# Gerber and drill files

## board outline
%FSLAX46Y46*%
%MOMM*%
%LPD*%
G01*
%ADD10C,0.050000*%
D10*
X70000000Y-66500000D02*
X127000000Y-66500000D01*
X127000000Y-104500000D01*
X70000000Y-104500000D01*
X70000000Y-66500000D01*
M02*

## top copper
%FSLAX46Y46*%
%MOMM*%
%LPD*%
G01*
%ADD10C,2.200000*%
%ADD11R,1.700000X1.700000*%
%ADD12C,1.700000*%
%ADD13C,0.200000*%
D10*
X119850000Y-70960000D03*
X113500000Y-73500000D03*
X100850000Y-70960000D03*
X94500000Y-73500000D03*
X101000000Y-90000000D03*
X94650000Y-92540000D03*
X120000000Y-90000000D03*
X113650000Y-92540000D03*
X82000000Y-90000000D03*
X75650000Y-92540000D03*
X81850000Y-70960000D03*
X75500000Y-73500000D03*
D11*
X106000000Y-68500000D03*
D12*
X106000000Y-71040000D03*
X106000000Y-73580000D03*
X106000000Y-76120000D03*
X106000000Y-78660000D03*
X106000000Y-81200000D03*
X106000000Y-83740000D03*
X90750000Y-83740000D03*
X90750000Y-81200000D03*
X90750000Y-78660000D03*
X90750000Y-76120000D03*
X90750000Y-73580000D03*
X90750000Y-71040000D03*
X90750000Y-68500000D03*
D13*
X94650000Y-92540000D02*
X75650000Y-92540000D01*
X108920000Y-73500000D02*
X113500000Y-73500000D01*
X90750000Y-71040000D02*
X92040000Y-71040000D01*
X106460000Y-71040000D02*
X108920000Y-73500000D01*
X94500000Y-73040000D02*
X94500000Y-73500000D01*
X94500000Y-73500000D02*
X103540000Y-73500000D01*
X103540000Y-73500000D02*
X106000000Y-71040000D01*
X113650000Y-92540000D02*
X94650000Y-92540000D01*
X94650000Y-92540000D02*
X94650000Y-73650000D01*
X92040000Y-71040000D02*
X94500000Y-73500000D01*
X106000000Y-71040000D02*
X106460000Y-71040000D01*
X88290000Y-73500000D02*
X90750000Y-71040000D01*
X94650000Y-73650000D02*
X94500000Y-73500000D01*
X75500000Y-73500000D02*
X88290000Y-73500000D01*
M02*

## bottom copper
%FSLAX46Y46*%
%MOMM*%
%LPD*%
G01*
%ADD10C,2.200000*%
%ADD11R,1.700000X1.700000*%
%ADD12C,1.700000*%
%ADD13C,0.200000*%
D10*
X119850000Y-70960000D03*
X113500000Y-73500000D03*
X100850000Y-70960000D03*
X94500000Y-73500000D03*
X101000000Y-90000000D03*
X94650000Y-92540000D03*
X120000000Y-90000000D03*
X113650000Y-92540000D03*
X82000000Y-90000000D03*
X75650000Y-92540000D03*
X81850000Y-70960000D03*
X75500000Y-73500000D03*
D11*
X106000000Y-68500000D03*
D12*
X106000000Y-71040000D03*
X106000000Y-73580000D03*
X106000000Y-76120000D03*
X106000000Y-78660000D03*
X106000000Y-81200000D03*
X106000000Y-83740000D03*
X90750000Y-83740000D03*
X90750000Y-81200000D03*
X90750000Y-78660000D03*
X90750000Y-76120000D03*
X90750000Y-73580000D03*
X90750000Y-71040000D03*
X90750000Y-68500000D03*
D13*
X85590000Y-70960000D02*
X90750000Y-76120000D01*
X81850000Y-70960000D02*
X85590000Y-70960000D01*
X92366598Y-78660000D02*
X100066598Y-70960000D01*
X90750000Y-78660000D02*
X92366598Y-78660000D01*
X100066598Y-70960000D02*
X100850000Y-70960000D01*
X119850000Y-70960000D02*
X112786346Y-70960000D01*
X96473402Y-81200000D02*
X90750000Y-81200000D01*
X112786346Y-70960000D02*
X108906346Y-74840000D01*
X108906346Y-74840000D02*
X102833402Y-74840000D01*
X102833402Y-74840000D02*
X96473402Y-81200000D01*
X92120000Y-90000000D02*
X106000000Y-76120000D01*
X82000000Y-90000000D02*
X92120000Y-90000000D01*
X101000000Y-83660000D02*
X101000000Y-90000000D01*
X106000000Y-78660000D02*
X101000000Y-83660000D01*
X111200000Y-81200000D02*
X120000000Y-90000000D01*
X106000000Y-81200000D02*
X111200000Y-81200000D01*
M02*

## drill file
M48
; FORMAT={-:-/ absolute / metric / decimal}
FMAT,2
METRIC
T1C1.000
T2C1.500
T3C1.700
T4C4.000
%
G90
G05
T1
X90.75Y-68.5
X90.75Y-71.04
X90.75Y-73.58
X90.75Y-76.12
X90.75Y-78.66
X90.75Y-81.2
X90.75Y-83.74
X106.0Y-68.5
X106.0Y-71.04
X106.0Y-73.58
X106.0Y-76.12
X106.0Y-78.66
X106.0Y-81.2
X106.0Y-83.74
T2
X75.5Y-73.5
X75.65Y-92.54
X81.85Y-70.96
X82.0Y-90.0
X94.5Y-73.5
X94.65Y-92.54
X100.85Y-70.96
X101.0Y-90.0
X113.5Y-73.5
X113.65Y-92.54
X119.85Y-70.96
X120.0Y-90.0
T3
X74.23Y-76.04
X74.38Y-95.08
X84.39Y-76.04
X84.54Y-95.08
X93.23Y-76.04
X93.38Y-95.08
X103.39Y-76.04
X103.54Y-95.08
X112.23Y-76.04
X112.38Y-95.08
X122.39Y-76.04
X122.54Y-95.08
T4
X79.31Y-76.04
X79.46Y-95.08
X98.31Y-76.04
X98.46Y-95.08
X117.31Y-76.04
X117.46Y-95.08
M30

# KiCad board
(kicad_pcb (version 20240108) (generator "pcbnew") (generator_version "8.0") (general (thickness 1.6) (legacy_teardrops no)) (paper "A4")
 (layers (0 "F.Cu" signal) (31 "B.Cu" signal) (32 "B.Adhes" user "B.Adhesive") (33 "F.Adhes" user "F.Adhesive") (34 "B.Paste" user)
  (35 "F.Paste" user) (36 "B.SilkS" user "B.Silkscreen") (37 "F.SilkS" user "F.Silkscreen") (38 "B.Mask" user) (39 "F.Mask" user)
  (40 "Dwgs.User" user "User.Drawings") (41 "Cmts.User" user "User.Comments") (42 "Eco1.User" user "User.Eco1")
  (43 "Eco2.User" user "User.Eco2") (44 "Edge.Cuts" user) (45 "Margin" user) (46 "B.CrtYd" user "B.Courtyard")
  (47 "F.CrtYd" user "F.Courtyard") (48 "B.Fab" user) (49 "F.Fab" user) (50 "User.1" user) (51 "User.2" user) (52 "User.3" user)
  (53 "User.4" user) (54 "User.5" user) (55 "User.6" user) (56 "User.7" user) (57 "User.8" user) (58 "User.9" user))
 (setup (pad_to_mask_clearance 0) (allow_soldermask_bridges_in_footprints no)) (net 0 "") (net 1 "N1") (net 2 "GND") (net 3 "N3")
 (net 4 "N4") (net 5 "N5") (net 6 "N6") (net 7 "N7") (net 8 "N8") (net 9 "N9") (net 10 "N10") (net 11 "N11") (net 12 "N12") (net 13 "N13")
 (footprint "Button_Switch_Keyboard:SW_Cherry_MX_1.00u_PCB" (layer "F.Cu") (at 119.85 70.96)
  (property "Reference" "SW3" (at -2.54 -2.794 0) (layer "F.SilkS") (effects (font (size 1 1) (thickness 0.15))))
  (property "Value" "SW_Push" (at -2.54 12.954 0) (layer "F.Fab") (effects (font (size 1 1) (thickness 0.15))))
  (pad "" np_thru_hole circle (at -7.62 5.08) (size 1.7 1.7) (drill 1.7) (layers "*.Cu" "*.Mask"))
  (pad "" np_thru_hole circle (at -2.54 5.08) (size 4 4) (drill 4) (layers "*.Cu" "*.Mask"))
  (pad "" np_thru_hole circle (at 2.54 5.08) (size 1.7 1.7) (drill 1.7) (layers "*.Cu" "*.Mask"))
  (pad "1" thru_hole circle (at 0 0) (size 2.2 2.2) (drill 1.5) (layers "*.Cu" "*.Mask") (remove_unused_layers no) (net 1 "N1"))
  (pad "2" thru_hole circle (at -6.35 2.54) (size 2.2 2.2) (drill 1.5) (layers "*.Cu" "*.Mask") (remove_unused_layers no) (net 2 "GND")))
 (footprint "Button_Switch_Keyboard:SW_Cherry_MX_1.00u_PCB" (layer "F.Cu") (at 100.85 70.96)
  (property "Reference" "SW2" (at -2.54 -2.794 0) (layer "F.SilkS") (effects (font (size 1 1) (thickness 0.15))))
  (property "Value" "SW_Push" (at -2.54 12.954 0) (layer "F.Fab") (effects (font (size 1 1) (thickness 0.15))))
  (pad "" np_thru_hole circle (at -7.62 5.08) (size 1.7 1.7) (drill 1.7) (layers "*.Cu" "*.Mask"))
  (pad "" np_thru_hole circle (at -2.54 5.08) (size 4 4) (drill 4) (layers "*.Cu" "*.Mask"))
  (pad "" np_thru_hole circle (at 2.54 5.08) (size 1.7 1.7) (drill 1.7) (layers "*.Cu" "*.Mask"))
  (pad "1" thru_hole circle (at 0 0) (size 2.2 2.2) (drill 1.5) (layers "*.Cu" "*.Mask") (remove_unused_layers no) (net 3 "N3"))
  (pad "2" thru_hole circle (at -6.35 2.54) (size 2.2 2.2) (drill 1.5) (layers "*.Cu" "*.Mask") (remove_unused_layers no) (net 2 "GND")))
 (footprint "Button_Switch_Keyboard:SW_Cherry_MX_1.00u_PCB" (layer "F.Cu") (at 101 90)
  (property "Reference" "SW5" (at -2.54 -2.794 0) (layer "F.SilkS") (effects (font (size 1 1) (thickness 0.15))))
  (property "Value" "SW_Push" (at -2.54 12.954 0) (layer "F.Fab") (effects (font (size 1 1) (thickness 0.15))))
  (pad "" np_thru_hole circle (at -7.62 5.08) (size 1.7 1.7) (drill 1.7) (layers "*.Cu" "*.Mask"))
  (pad "" np_thru_hole circle (at -2.54 5.08) (size 4 4) (drill 4) (layers "*.Cu" "*.Mask"))
  (pad "" np_thru_hole circle (at 2.54 5.08) (size 1.7 1.7) (drill 1.7) (layers "*.Cu" "*.Mask"))
  (pad "1" thru_hole circle (at 0 0) (size 2.2 2.2) (drill 1.5) (layers "*.Cu" "*.Mask") (remove_unused_layers no) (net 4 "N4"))
  (pad "2" thru_hole circle (at -6.35 2.54) (size 2.2 2.2) (drill 1.5) (layers "*.Cu" "*.Mask") (remove_unused_layers no) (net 2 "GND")))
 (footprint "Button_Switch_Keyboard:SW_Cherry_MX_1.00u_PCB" (layer "F.Cu") (at 120 90)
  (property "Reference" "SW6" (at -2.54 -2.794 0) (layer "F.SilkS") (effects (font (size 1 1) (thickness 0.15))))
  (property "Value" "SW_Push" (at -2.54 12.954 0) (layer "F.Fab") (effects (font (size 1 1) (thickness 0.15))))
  (pad "" np_thru_hole circle (at -7.62 5.08) (size 1.7 1.7) (drill 1.7) (layers "*.Cu" "*.Mask"))
  (pad "" np_thru_hole circle (at -2.54 5.08) (size 4 4) (drill 4) (layers "*.Cu" "*.Mask"))
  (pad "" np_thru_hole circle (at 2.54 5.08) (size 1.7 1.7) (drill 1.7) (layers "*.Cu" "*.Mask"))
  (pad "1" thru_hole circle (at 0 0) (size 2.2 2.2) (drill 1.5) (layers "*.Cu" "*.Mask") (remove_unused_layers no) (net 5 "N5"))
  (pad "2" thru_hole circle (at -6.35 2.54) (size 2.2 2.2) (drill 1.5) (layers "*.Cu" "*.Mask") (remove_unused_layers no) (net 2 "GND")))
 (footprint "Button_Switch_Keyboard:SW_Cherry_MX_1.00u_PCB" (layer "F.Cu") (at 82 90)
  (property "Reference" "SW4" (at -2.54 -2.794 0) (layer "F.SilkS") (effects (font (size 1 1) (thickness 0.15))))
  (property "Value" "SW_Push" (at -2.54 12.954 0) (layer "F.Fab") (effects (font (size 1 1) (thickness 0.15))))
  (pad "" np_thru_hole circle (at -7.62 5.08) (size 1.7 1.7) (drill 1.7) (layers "*.Cu" "*.Mask"))
  (pad "" np_thru_hole circle (at -2.54 5.08) (size 4 4) (drill 4) (layers "*.Cu" "*.Mask"))
  (pad "" np_thru_hole circle (at 2.54 5.08) (size 1.7 1.7) (drill 1.7) (layers "*.Cu" "*.Mask"))
  (pad "1" thru_hole circle (at 0 0) (size 2.2 2.2) (drill 1.5) (layers "*.Cu" "*.Mask") (remove_unused_layers no) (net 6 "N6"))
  (pad "2" thru_hole circle (at -6.35 2.54) (size 2.2 2.2) (drill 1.5) (layers "*.Cu" "*.Mask") (remove_unused_layers no) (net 2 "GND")))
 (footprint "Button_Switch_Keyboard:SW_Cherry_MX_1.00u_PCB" (layer "F.Cu") (at 81.85 70.96)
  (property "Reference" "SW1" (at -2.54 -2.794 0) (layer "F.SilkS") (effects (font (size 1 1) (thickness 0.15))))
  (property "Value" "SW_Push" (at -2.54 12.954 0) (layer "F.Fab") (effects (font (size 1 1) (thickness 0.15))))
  (pad "" np_thru_hole circle (at -7.62 5.08) (size 1.7 1.7) (drill 1.7) (layers "*.Cu" "*.Mask"))
  (pad "" np_thru_hole circle (at -2.54 5.08) (size 4 4) (drill 4) (layers "*.Cu" "*.Mask"))
  (pad "" np_thru_hole circle (at 2.54 5.08) (size 1.7 1.7) (drill 1.7) (layers "*.Cu" "*.Mask"))
  (pad "1" thru_hole circle (at 0 0) (size 2.2 2.2) (drill 1.5) (layers "*.Cu" "*.Mask") (remove_unused_layers no) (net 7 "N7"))
  (pad "2" thru_hole circle (at -6.35 2.54) (size 2.2 2.2) (drill 1.5) (layers "*.Cu" "*.Mask") (remove_unused_layers no) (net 2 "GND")))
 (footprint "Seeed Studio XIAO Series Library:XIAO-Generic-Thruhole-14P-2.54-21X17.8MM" (layer "B.Cu") (at 98.375 76.12 180)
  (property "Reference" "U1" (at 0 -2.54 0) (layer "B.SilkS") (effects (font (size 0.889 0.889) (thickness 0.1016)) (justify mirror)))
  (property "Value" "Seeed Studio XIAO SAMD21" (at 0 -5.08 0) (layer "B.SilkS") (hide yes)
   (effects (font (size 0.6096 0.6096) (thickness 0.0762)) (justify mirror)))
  (pad "1" thru_hole rect (at -7.625 7.62 180) (size 1.7 1.7) (drill 1) (layers "*.Cu" "*.Mask") (remove_unused_layers no) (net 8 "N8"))
  (pad "2" thru_hole circle (at -7.625 5.08 180) (size 1.7 1.7) (drill 1) (layers "*.Cu" "*.Mask") (remove_unused_layers no) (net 2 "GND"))
  (pad "3" thru_hole circle (at -7.625 2.54 180) (size 1.7 1.7) (drill 1) (layers "*.Cu" "*.Mask") (remove_unused_layers no) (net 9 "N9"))
  (pad "4" thru_hole circle (at -7.625 0 180) (size 1.7 1.7) (drill 1) (layers "*.Cu" "*.Mask") (remove_unused_layers no) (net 6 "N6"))
  (pad "5" thru_hole circle (at -7.625 -2.54 180) (size 1.7 1.7) (drill 1) (layers "*.Cu" "*.Mask") (remove_unused_layers no) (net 4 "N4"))
  (pad "6" thru_hole circle (at -7.625 -5.08) (size 1.7 1.7) (drill 1) (layers "*.Cu" "*.Mask") (remove_unused_layers no) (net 5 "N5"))
  (pad "7" thru_hole circle (at -7.625 -7.62 180) (size 1.7 1.7) (drill 1) (layers "*.Cu" "*.Mask") (remove_unused_layers no) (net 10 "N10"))
  (pad "8" thru_hole circle (at 7.625 -7.62 180) (size 1.7 1.7) (drill 1) (layers "*.Cu" "*.Mask") (remove_unused_layers no) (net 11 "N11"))
  (pad "9" thru_hole circle (at 7.625 -5.08 180) (size 1.7 1.7) (drill 1) (layers "*.Cu" "*.Mask") (remove_unused_layers no) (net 1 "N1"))
  (pad "10" thru_hole circle (at 7.625 -2.54 180) (size 1.7 1.7) (drill 1) (layers "*.Cu" "*.Mask") (remove_unused_layers no) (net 3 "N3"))
  (pad "11" thru_hole circle (at 7.625 0 180) (size 1.7 1.7) (drill 1) (layers "*.Cu" "*.Mask") (remove_unused_layers no) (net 7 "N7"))
  (pad "12" thru_hole circle (at 7.625 2.54 180) (size 1.7 1.7) (drill 1) (layers "*.Cu" "*.Mask") (remove_unused_layers no) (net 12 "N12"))
  (pad "13" thru_hole circle (at 7.625 5.08 180) (size 1.7 1.7) (drill 1) (layers "*.Cu" "*.Mask") (remove_unused_layers no) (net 2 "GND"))
  (pad "14" thru_hole circle (at 7.625 7.62 180) (size 1.7 1.7) (drill 1) (layers "*.Cu" "*.Mask") (remove_unused_layers no) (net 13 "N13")))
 (gr_rect (start 70 66.5) (end 127 104.5) (stroke (width 0.05) (type default)) (fill none) (layer "Edge.Cuts"))
 (segment (start 94.65 92.54) (end 75.65 92.54) (width 0.2) (layer "F.Cu") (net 2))
 (segment (start 108.92 73.5) (end 113.5 73.5) (width 0.2) (layer "F.Cu") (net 2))
 (segment (start 90.75 71.04) (end 92.04 71.04) (width 0.2) (layer "F.Cu") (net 2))
 (segment (start 106.46 71.04) (end 108.92 73.5) (width 0.2) (layer "F.Cu") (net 2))
 (segment (start 94.5 73.04) (end 94.5 73.5) (width 0.2) (layer "F.Cu") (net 2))
 (segment (start 94.5 73.5) (end 103.54 73.5) (width 0.2) (layer "F.Cu") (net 2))
 (segment (start 103.54 73.5) (end 106 71.04) (width 0.2) (layer "F.Cu") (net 2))
 (segment (start 113.65 92.54) (end 94.65 92.54) (width 0.2) (layer "F.Cu") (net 2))
 (segment (start 94.65 92.54) (end 94.65 73.65) (width 0.2) (layer "F.Cu") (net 2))
 (segment (start 92.04 71.04) (end 94.5 73.5) (width 0.2) (layer "F.Cu") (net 2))
 (segment (start 106 71.04) (end 106.46 71.04) (width 0.2) (layer "F.Cu") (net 2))
 (segment (start 88.29 73.5) (end 90.75 71.04) (width 0.2) (layer "F.Cu") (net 2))
 (segment (start 94.65 73.65) (end 94.5 73.5) (width 0.2) (layer "F.Cu") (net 2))
 (segment (start 75.5 73.5) (end 88.29 73.5) (width 0.2) (layer "F.Cu") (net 2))
 (segment (start 85.59 70.96) (end 90.75 76.12) (width 0.2) (layer "B.Cu") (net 7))
 (segment (start 81.85 70.96) (end 85.59 70.96) (width 0.2) (layer "B.Cu") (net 7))
 (segment (start 92.366598 78.66) (end 100.066598 70.96) (width 0.2) (layer "B.Cu") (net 3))
 (segment (start 90.75 78.66) (end 92.366598 78.66) (width 0.2) (layer "B.Cu") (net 3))
 (segment (start 100.066598 70.96) (end 100.85 70.96) (width 0.2) (layer "B.Cu") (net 3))
 (segment (start 119.85 70.96) (end 112.786346 70.96) (width 0.2) (layer "B.Cu") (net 1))
 (segment (start 96.473402 81.2) (end 90.75 81.2) (width 0.2) (layer "B.Cu") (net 1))
 (segment (start 112.786346 70.96) (end 108.906346 74.84) (width 0.2) (layer "B.Cu") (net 1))
 (segment (start 108.906346 74.84) (end 102.833402 74.84) (width 0.2) (layer "B.Cu") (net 1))
 (segment (start 102.833402 74.84) (end 96.473402 81.2) (width 0.2) (layer "B.Cu") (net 1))
 (segment (start 92.12 90) (end 106 76.12) (width 0.2) (layer "B.Cu") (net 6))
 (segment (start 82 90) (end 92.12 90) (width 0.2) (layer "B.Cu") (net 6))
 (segment (start 101 83.66) (end 101 90) (width 0.2) (layer "B.Cu") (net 4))
 (segment (start 106 78.66) (end 101 83.66) (width 0.2) (layer "B.Cu") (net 4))
 (segment (start 111.2 81.2) (end 120 90) (width 0.2) (layer "B.Cu") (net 5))
 (segment (start 106 81.2) (end 111.2 81.2) (width 0.2) (layer "B.Cu") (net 5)))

